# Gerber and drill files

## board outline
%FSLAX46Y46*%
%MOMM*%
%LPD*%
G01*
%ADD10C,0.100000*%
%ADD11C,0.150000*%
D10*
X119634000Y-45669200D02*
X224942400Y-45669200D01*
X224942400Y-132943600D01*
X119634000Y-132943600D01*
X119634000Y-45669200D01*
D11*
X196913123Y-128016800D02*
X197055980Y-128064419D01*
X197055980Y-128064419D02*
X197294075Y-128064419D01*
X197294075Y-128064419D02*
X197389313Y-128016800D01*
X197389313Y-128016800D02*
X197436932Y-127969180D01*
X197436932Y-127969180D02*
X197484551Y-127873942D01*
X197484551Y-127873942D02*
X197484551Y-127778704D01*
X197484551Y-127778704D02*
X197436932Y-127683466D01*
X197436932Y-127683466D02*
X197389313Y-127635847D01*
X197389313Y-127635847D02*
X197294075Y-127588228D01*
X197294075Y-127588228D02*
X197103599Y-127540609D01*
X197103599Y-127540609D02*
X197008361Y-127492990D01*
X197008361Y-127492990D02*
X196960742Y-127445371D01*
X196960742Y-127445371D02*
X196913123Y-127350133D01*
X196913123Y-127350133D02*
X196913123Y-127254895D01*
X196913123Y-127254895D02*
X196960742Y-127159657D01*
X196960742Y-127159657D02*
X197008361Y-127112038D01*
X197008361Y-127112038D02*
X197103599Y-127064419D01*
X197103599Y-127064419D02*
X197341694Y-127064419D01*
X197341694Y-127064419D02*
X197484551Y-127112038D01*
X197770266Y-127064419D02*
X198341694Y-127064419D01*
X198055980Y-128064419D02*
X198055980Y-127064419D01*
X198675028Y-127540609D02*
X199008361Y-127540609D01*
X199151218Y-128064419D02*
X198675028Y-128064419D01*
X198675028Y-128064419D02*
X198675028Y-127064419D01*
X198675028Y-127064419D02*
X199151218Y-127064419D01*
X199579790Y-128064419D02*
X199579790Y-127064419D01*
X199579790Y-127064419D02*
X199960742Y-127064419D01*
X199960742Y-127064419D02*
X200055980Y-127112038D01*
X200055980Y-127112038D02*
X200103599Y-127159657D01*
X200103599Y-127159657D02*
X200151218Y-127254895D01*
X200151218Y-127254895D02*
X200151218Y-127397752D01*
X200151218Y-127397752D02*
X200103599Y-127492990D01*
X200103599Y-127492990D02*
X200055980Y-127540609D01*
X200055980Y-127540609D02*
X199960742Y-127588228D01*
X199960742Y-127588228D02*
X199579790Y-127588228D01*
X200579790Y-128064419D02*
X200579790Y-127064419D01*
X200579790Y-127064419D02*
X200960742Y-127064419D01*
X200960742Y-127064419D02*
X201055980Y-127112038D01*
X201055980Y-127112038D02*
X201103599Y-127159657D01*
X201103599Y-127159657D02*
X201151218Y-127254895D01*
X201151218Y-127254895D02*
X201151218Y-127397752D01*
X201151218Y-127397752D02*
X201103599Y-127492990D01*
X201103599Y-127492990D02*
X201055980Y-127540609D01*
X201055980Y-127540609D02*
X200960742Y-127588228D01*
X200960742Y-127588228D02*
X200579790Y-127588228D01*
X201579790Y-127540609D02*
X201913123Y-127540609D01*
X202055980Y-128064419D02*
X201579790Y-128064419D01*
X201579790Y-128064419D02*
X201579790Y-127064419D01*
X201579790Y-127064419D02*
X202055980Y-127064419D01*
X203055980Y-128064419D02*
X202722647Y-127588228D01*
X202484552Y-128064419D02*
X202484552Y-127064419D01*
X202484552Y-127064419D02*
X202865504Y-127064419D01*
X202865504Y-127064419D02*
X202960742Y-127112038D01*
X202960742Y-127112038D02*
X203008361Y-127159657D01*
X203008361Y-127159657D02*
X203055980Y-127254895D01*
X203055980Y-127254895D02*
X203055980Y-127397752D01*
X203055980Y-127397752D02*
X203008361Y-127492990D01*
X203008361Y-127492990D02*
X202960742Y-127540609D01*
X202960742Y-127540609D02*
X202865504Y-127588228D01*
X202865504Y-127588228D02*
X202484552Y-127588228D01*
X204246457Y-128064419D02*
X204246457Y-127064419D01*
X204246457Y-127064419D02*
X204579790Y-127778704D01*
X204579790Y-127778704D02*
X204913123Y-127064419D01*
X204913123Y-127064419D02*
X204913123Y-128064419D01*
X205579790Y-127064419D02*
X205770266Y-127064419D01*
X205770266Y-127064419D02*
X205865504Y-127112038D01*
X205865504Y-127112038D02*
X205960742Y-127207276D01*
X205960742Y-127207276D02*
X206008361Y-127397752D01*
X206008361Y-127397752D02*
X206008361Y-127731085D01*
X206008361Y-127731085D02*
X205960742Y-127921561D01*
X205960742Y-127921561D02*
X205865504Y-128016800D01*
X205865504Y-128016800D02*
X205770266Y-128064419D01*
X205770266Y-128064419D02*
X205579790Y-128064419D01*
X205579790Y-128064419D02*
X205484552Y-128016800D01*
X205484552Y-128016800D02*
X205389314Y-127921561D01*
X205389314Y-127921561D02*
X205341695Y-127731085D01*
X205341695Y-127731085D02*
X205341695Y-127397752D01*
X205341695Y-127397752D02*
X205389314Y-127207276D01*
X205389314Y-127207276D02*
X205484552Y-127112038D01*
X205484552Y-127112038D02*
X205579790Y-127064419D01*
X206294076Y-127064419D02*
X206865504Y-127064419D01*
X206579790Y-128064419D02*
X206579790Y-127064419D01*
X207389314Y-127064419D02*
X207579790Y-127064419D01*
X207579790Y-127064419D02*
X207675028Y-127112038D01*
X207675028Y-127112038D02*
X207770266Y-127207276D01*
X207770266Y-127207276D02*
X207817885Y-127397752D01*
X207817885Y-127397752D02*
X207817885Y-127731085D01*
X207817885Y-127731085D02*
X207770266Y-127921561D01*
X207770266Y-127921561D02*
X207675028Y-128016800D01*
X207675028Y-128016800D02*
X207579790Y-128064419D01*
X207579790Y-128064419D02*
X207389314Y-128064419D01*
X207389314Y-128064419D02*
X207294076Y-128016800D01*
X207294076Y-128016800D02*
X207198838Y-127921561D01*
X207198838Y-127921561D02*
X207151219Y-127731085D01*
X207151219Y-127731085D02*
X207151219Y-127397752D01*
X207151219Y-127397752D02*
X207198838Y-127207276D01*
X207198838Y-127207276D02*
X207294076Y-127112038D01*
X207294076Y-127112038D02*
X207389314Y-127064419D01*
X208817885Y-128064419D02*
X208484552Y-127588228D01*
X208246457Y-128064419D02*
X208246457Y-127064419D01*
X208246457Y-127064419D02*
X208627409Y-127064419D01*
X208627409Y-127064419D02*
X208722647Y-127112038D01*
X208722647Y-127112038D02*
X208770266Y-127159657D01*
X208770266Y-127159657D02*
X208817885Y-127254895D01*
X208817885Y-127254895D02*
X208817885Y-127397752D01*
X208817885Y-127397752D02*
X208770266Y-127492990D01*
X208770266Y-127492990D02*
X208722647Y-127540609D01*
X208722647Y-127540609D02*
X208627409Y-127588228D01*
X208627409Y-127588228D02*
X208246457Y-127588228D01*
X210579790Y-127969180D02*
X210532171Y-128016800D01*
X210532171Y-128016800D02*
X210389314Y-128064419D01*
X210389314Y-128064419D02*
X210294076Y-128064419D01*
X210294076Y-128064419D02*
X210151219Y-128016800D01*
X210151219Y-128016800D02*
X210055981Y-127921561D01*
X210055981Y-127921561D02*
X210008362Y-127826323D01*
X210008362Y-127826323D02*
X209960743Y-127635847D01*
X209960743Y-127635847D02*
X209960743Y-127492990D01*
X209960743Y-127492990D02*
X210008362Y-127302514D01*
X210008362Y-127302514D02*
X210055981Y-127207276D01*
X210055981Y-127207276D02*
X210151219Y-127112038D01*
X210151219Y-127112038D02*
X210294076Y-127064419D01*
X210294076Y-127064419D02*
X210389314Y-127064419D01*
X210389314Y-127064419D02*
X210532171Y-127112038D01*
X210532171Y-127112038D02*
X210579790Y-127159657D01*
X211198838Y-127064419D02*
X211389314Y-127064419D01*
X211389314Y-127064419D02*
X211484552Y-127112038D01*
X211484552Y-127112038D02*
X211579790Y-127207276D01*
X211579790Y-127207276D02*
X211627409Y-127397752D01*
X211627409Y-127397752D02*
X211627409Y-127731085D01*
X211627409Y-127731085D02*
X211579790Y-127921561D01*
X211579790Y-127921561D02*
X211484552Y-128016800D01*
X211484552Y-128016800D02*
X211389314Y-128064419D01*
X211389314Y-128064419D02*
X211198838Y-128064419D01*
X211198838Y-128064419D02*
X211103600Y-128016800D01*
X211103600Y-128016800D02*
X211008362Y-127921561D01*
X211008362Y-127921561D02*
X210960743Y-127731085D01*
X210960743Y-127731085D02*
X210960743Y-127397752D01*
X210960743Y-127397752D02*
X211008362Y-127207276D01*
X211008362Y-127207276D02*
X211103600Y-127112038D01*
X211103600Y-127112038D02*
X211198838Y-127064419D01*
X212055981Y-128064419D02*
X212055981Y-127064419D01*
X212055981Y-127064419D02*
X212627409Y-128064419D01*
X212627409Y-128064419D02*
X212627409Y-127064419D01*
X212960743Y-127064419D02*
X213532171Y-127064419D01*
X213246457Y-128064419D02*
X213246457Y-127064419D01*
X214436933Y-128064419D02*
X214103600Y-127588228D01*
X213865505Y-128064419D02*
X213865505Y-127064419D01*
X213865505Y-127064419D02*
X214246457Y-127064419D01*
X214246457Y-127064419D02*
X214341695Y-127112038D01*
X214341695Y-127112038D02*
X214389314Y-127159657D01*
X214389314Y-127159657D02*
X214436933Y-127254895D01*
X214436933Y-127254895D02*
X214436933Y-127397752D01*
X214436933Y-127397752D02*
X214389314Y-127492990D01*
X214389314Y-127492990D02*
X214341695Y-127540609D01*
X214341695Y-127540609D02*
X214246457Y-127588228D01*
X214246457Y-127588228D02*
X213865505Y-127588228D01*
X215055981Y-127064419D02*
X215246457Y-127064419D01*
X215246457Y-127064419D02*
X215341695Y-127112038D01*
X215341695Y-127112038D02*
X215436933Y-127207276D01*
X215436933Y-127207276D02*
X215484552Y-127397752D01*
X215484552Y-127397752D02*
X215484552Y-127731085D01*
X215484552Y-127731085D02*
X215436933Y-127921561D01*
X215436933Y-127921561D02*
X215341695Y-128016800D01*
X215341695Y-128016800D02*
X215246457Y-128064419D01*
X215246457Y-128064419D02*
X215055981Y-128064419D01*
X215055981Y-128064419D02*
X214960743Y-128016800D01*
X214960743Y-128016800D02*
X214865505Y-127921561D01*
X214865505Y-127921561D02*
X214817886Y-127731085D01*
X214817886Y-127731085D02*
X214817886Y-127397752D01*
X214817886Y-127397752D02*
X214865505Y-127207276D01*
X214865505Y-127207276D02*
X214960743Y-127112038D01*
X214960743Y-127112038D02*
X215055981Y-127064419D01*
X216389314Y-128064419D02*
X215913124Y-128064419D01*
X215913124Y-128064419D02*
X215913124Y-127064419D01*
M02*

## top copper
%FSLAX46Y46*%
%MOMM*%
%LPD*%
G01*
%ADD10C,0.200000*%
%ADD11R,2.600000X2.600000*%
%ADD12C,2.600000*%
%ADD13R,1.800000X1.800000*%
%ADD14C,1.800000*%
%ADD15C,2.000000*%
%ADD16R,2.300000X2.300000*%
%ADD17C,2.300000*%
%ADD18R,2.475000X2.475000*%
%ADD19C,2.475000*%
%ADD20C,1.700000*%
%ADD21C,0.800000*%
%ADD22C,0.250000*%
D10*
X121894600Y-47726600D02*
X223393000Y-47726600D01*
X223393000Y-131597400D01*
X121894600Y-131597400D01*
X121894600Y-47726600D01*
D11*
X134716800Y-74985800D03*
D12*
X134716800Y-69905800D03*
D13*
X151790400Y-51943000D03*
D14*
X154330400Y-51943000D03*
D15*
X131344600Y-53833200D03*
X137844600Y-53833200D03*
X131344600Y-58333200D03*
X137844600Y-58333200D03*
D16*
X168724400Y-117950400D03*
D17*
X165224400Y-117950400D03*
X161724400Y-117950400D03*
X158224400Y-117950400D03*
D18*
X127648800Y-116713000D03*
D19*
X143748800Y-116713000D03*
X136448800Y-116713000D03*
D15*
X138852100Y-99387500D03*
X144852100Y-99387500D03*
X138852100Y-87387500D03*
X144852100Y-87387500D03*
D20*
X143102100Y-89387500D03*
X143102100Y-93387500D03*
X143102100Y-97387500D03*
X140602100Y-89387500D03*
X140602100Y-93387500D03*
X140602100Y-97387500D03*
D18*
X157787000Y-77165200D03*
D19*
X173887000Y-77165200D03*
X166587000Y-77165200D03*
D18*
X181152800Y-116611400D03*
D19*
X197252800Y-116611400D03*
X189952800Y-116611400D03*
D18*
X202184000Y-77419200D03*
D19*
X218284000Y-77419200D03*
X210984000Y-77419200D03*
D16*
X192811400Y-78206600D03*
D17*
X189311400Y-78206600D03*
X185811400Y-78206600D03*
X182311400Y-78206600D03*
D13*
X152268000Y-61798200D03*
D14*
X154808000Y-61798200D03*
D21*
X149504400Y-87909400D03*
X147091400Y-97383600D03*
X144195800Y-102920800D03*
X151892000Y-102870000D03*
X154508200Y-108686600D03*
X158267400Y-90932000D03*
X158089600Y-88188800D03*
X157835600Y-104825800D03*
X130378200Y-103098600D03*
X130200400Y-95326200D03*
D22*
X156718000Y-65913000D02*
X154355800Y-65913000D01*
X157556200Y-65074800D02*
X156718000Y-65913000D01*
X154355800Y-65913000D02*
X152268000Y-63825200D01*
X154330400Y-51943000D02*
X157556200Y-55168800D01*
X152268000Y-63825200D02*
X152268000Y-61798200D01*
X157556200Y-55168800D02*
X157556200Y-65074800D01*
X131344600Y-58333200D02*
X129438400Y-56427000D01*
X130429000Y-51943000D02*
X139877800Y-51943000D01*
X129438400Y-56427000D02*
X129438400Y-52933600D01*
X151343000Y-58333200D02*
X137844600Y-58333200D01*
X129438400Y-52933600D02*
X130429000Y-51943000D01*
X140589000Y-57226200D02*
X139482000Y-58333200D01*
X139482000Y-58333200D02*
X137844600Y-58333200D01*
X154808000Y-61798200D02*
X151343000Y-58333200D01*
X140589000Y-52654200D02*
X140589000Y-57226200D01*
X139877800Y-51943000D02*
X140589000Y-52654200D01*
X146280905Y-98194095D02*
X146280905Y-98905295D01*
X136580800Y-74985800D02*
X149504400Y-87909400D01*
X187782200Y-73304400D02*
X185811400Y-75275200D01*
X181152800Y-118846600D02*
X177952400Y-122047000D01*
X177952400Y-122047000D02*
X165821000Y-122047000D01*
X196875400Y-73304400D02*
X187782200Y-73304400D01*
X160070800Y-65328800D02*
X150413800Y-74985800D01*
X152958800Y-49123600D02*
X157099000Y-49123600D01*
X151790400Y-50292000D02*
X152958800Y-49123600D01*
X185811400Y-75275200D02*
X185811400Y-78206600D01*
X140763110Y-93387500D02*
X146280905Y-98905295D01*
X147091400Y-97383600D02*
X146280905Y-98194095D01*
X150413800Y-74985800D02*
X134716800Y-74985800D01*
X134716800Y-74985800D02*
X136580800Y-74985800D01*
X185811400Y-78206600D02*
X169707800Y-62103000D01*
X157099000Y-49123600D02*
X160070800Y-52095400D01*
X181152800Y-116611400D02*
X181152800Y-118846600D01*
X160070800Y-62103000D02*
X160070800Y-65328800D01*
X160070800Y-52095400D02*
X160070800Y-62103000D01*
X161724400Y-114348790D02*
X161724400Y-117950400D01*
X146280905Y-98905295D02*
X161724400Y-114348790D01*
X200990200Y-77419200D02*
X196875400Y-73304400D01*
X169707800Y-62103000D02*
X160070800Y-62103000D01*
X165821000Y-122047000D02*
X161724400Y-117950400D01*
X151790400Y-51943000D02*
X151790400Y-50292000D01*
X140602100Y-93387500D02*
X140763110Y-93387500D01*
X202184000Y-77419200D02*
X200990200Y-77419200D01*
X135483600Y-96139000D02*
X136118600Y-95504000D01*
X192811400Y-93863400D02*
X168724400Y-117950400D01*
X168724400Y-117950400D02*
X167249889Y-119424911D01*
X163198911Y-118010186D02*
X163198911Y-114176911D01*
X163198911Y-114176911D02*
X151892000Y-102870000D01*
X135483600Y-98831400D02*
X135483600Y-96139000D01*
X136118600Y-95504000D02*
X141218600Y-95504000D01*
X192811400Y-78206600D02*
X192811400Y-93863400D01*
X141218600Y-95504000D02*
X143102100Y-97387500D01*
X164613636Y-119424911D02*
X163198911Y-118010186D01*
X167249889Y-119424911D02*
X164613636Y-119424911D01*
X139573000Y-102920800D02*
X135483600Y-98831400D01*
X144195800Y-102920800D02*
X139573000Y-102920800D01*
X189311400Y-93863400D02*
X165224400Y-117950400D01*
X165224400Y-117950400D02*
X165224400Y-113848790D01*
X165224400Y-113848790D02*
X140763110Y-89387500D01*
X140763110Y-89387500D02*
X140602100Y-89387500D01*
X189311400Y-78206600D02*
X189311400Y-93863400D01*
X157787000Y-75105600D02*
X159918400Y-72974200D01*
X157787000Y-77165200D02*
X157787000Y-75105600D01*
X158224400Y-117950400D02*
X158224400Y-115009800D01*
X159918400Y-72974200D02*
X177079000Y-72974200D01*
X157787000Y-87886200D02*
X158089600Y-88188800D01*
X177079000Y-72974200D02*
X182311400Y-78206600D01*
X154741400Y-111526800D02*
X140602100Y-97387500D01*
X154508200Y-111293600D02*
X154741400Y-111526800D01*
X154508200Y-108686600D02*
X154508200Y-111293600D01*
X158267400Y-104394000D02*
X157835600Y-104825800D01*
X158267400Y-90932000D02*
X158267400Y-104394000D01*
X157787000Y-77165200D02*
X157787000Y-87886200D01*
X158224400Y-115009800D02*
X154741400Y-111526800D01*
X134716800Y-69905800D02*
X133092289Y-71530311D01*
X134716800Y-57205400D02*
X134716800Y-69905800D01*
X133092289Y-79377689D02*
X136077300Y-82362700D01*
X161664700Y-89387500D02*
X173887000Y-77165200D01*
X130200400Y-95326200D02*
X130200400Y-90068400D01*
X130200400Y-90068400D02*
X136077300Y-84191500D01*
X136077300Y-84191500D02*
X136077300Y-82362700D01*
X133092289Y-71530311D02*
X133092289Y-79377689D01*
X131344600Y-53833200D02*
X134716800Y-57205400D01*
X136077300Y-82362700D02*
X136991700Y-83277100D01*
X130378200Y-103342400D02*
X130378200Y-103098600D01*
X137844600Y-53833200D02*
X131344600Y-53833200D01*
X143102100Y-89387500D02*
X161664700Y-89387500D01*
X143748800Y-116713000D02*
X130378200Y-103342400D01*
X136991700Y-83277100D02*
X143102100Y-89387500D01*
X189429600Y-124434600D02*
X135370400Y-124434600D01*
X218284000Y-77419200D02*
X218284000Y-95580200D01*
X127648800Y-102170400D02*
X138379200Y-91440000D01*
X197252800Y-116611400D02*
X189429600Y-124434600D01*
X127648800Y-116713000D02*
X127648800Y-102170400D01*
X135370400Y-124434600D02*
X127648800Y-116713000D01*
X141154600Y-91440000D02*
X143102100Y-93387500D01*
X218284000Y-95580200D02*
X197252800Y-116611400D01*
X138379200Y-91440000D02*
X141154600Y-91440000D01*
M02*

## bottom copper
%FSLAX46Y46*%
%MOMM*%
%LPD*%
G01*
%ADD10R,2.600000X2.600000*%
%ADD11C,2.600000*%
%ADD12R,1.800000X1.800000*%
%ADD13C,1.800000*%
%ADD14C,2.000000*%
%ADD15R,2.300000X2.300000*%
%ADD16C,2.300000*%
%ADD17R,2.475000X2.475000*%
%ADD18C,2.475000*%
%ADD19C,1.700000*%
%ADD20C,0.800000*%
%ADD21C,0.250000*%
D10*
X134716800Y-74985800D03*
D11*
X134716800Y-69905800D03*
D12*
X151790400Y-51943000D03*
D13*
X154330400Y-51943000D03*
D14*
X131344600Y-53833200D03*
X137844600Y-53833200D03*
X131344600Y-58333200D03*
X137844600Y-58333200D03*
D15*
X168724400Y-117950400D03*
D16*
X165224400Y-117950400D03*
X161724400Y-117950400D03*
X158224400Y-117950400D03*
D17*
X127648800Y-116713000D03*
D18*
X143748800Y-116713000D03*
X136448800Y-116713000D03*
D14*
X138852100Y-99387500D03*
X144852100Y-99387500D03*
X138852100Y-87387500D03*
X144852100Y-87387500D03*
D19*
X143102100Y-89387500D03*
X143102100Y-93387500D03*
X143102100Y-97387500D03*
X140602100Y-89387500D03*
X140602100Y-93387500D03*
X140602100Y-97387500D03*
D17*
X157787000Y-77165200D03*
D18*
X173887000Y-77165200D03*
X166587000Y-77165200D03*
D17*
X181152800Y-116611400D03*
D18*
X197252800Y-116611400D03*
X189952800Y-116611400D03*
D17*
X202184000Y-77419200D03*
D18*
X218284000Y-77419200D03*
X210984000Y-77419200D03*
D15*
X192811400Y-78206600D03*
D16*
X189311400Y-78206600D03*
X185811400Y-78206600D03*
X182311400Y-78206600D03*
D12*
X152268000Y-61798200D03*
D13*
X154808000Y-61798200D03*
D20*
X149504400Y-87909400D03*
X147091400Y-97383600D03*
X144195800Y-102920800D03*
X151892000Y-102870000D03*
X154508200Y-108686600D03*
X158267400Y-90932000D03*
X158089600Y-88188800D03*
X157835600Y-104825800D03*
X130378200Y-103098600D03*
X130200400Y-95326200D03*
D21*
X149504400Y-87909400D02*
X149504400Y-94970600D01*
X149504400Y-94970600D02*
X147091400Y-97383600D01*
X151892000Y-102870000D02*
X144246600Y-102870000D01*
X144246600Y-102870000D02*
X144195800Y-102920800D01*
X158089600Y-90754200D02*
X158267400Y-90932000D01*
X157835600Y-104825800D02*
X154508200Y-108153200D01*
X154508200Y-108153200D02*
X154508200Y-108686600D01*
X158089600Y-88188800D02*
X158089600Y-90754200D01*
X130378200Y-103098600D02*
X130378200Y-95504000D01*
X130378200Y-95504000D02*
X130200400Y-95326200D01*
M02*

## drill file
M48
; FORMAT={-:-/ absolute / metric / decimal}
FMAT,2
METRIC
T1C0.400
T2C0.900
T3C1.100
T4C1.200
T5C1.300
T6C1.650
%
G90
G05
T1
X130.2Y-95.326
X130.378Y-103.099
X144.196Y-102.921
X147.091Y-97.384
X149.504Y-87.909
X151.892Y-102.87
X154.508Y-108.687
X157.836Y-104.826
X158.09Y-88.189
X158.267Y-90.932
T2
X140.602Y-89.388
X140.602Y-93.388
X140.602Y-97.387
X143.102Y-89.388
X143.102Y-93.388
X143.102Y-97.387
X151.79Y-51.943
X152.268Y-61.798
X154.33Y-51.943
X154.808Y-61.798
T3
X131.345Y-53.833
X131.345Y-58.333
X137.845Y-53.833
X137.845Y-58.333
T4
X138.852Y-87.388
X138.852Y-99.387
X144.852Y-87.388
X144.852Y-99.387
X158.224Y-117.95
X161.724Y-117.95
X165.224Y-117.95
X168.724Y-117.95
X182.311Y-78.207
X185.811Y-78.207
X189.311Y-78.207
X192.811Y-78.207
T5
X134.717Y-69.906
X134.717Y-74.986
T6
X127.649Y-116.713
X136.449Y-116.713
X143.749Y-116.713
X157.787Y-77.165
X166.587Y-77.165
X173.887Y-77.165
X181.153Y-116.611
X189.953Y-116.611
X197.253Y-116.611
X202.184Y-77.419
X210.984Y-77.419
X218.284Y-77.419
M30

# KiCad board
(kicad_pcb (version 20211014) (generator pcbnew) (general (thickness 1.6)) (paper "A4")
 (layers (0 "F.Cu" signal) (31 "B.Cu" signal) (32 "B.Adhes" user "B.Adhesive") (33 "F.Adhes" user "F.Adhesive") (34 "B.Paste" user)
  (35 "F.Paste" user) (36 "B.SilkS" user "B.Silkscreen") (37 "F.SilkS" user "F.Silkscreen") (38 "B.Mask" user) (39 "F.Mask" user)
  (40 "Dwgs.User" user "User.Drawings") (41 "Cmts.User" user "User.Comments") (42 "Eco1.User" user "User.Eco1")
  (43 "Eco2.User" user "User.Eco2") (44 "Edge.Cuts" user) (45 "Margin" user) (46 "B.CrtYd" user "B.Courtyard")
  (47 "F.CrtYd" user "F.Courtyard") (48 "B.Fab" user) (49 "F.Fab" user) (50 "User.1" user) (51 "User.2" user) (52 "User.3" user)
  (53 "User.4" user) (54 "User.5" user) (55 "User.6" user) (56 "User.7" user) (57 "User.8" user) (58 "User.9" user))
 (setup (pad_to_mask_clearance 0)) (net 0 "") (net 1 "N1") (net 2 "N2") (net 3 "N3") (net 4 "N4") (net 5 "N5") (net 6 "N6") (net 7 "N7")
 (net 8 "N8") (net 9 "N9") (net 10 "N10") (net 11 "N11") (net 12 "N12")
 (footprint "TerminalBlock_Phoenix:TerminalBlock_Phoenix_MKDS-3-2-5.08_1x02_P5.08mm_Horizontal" (layer "F.Cu") (at 134.7168 74.9858 90)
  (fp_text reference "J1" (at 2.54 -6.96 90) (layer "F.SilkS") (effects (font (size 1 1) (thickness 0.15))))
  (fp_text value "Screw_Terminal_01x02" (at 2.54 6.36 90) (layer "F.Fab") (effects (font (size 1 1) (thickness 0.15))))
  (pad "1" thru_hole rect (at 0 0 90) (size 2.6 2.6) (drill 1.3) (layers *.Cu *.Mask) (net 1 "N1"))
  (pad "2" thru_hole circle (at 5.08 0 90) (size 2.6 2.6) (drill 1.3) (layers *.Cu *.Mask) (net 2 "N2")))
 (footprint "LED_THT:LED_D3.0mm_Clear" (layer "F.Cu") (at 151.7904 51.943)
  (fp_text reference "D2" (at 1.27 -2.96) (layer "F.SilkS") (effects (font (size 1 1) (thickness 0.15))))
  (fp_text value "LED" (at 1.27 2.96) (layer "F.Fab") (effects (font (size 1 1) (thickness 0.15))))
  (pad "1" thru_hole rect (at 0 0) (size 1.8 1.8) (drill 0.9) (layers *.Cu *.Mask) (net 1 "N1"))
  (pad "2" thru_hole circle (at 2.54 0) (size 1.8 1.8) (drill 0.9) (layers *.Cu *.Mask) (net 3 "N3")))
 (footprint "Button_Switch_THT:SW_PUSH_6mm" (layer "F.Cu") (at 131.3446 53.8332)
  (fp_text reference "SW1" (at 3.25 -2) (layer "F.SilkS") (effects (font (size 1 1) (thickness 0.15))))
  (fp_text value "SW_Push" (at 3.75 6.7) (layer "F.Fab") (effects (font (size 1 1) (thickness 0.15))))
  (pad "1" thru_hole circle (at 0 0 90) (size 2 2) (drill 1.1) (layers *.Cu *.Mask) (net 2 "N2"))
  (pad "1" thru_hole circle (at 6.5 0 90) (size 2 2) (drill 1.1) (layers *.Cu *.Mask) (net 2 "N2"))
  (pad "2" thru_hole circle (at 0 4.5 90) (size 2 2) (drill 1.1) (layers *.Cu *.Mask) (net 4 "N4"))
  (pad "2" thru_hole circle (at 6.5 4.5 90) (size 2 2) (drill 1.1) (layers *.Cu *.Mask) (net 4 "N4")))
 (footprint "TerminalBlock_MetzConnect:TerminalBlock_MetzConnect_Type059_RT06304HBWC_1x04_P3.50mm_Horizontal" (layer "F.Cu")
  (at 168.7244 117.9504 180)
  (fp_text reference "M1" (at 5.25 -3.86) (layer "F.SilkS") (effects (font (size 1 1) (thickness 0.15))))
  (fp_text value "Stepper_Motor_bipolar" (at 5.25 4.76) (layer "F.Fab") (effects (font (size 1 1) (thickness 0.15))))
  (pad "1" thru_hole rect (at 0 0 180) (size 2.3 2.3) (drill 1.2) (layers *.Cu *.Mask) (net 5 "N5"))
  (pad "2" thru_hole circle (at 3.5 0 180) (size 2.3 2.3) (drill 1.2) (layers *.Cu *.Mask) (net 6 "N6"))
  (pad "3" thru_hole circle (at 7 0 180) (size 2.3 2.3) (drill 1.2) (layers *.Cu *.Mask) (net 1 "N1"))
  (pad "4" thru_hole circle (at 10.5 0 180) (size 2.3 2.3) (drill 1.2) (layers *.Cu *.Mask) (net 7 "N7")))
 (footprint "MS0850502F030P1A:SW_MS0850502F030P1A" (layer "F.Cu") (at 127.6488 116.713)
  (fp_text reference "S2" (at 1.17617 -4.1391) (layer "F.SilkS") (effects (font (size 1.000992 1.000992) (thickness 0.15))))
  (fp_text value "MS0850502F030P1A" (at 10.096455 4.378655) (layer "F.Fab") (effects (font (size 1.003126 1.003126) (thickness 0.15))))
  (pad "1" thru_hole rect (at 0 0) (size 2.475 2.475) (drill 1.65) (layers *.Cu *.Mask) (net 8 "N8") (solder_mask_margin 0.102))
  (pad "2" thru_hole circle (at 16.1 0) (size 2.475 2.475) (drill 1.65) (layers *.Cu *.Mask) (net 2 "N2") (solder_mask_margin 0.102))
  (pad "3" thru_hole circle (at 8.8 0) (size 2.475 2.475) (drill 1.65) (layers *.Cu *.Mask) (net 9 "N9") (solder_mask_margin 0.102)))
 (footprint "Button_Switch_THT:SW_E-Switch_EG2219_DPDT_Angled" (layer "F.Cu") (at 143.1021 89.3875 -90)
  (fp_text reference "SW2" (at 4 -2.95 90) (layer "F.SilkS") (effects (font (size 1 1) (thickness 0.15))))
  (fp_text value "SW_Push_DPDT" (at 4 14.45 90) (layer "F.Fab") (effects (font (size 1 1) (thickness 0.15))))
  (pad "" thru_hole circle (at 10 4.25 270) (size 2 2) (drill 1.2) (layers *.Cu *.Mask))
  (pad "" thru_hole circle (at 10 -1.75 270) (size 2 2) (drill 1.2) (layers *.Cu *.Mask))
  (pad "" thru_hole circle (at -2 4.25 270) (size 2 2) (drill 1.2) (layers *.Cu *.Mask))
  (pad "" thru_hole circle (at -2 -1.75 270) (size 2 2) (drill 1.2) (layers *.Cu *.Mask))
  (pad "1" thru_hole circle (at 0 0 270) (size 1.7 1.7) (drill 0.9) (layers *.Cu *.Mask) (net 2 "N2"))
  (pad "2" thru_hole circle (at 4 0 270) (size 1.7 1.7) (drill 0.9) (layers *.Cu *.Mask) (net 8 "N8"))
  (pad "3" thru_hole circle (at 8 0 270) (size 1.7 1.7) (drill 0.9) (layers *.Cu *.Mask) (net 5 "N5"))
  (pad "4" thru_hole circle (at 0 2.5 270) (size 1.7 1.7) (drill 0.9) (layers *.Cu *.Mask) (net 6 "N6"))
  (pad "5" thru_hole circle (at 4 2.5 270) (size 1.7 1.7) (drill 0.9) (layers *.Cu *.Mask) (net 1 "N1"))
  (pad "6" thru_hole circle (at 8 2.5 270) (size 1.7 1.7) (drill 0.9) (layers *.Cu *.Mask) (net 7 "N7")))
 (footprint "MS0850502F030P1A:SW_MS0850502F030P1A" (layer "F.Cu") (at 157.787 77.1652)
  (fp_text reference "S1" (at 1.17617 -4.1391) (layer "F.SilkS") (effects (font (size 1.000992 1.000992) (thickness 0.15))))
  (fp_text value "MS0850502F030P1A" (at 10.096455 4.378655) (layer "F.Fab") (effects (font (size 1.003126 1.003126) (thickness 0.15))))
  (pad "1" thru_hole rect (at 0 0) (size 2.475 2.475) (drill 1.65) (layers *.Cu *.Mask) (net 7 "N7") (solder_mask_margin 0.102))
  (pad "2" thru_hole circle (at 16.1 0) (size 2.475 2.475) (drill 1.65) (layers *.Cu *.Mask) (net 2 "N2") (solder_mask_margin 0.102))
  (pad "3" thru_hole circle (at 8.8 0) (size 2.475 2.475) (drill 1.65) (layers *.Cu *.Mask) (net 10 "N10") (solder_mask_margin 0.102)))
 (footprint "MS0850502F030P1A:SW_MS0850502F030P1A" (layer "F.Cu") (at 181.1528 116.6114)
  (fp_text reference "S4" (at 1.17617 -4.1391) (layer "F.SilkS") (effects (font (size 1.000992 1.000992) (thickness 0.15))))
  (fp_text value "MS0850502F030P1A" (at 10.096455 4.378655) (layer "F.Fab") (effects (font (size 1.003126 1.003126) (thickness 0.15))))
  (pad "1" thru_hole rect (at 0 0) (size 2.475 2.475) (drill 1.65) (layers *.Cu *.Mask) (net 1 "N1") (solder_mask_margin 0.102))
  (pad "2" thru_hole circle (at 16.1 0) (size 2.475 2.475) (drill 1.65) (layers *.Cu *.Mask) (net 8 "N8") (solder_mask_margin 0.102))
  (pad "3" thru_hole circle (at 8.8 0) (size 2.475 2.475) (drill 1.65) (layers *.Cu *.Mask) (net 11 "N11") (solder_mask_margin 0.102)))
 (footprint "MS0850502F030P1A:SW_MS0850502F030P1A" (layer "F.Cu") (at 202.184 77.4192)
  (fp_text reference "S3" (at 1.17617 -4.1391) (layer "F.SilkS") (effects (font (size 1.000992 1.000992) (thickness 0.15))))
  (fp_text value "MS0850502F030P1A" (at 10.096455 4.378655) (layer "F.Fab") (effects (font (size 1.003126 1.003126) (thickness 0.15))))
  (pad "1" thru_hole rect (at 0 0) (size 2.475 2.475) (drill 1.65) (layers *.Cu *.Mask) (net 1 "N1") (solder_mask_margin 0.102))
  (pad "2" thru_hole circle (at 16.1 0) (size 2.475 2.475) (drill 1.65) (layers *.Cu *.Mask) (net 8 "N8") (solder_mask_margin 0.102))
  (pad "3" thru_hole circle (at 8.8 0) (size 2.475 2.475) (drill 1.65) (layers *.Cu *.Mask) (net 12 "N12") (solder_mask_margin 0.102)))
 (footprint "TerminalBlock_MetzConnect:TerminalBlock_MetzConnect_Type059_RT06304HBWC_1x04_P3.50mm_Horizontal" (layer "F.Cu")
  (at 192.8114 78.2066 180)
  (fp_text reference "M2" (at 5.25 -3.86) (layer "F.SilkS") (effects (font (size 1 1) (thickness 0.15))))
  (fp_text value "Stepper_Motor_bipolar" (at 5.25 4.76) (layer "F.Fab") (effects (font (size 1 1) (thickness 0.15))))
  (pad "1" thru_hole rect (at 0 0 180) (size 2.3 2.3) (drill 1.2) (layers *.Cu *.Mask) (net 5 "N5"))
  (pad "2" thru_hole circle (at 3.5 0 180) (size 2.3 2.3) (drill 1.2) (layers *.Cu *.Mask) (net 6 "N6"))
  (pad "3" thru_hole circle (at 7 0 180) (size 2.3 2.3) (drill 1.2) (layers *.Cu *.Mask) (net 1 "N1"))
  (pad "4" thru_hole circle (at 10.5 0 180) (size 2.3 2.3) (drill 1.2) (layers *.Cu *.Mask) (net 7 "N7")))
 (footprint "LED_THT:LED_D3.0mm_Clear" (layer "F.Cu") (at 152.268 61.7982)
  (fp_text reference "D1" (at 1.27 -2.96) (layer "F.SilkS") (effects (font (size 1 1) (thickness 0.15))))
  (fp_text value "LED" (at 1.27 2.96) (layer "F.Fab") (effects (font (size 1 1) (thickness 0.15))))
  (pad "1" thru_hole rect (at 0 0) (size 1.8 1.8) (drill 0.9) (layers *.Cu *.Mask) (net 3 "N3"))
  (pad "2" thru_hole circle (at 2.54 0) (size 1.8 1.8) (drill 0.9) (layers *.Cu *.Mask) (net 4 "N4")))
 (gr_rect (start 121.8946 47.7266) (end 223.393 131.5974) (layer "F.Cu") (width 0.2) (fill none))
 (gr_rect (start 119.634 45.6692) (end 224.9424 132.9436) (layer "Edge.Cuts") (width 0.1) (fill none))
 (gr_rect (start 224.9424 132.9436) (end 224.9424 132.9436) (layer "Edge.Cuts") (width 0.1) (fill none))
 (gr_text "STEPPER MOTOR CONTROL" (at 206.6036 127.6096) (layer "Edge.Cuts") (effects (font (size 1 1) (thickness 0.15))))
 (segment (start 156.718 65.913) (end 154.3558 65.913) (width 0.25) (layer "F.Cu") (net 3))
 (segment (start 157.5562 65.0748) (end 156.718 65.913) (width 0.25) (layer "F.Cu") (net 3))
 (segment (start 154.3558 65.913) (end 152.268 63.8252) (width 0.25) (layer "F.Cu") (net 3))
 (segment (start 154.3304 51.943) (end 157.5562 55.1688) (width 0.25) (layer "F.Cu") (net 3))
 (segment (start 152.268 63.8252) (end 152.268 61.7982) (width 0.25) (layer "F.Cu") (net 3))
 (segment (start 157.5562 55.1688) (end 157.5562 65.0748) (width 0.25) (layer "F.Cu") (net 3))
 (segment (start 131.3446 58.3332) (end 129.4384 56.427) (width 0.25) (layer "F.Cu") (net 4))
 (segment (start 130.429 51.943) (end 139.8778 51.943) (width 0.25) (layer "F.Cu") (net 4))
 (segment (start 129.4384 56.427) (end 129.4384 52.9336) (width 0.25) (layer "F.Cu") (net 4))
 (segment (start 151.343 58.3332) (end 137.8446 58.3332) (width 0.25) (layer "F.Cu") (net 4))
 (segment (start 129.4384 52.9336) (end 130.429 51.943) (width 0.25) (layer "F.Cu") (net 4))
 (segment (start 140.589 57.2262) (end 139.482 58.3332) (width 0.25) (layer "F.Cu") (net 4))
 (segment (start 139.482 58.3332) (end 137.8446 58.3332) (width 0.25) (layer "F.Cu") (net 4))
 (segment (start 154.808 61.7982) (end 151.343 58.3332) (width 0.25) (layer "F.Cu") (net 4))
 (segment (start 140.589 52.6542) (end 140.589 57.2262) (width 0.25) (layer "F.Cu") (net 4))
 (segment (start 139.8778 51.943) (end 140.589 52.6542) (width 0.25) (layer "F.Cu") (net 4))
 (segment (start 146.280905 98.194095) (end 146.280905 98.905295) (width 0.25) (layer "F.Cu") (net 1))
 (segment (start 136.5808 74.9858) (end 149.5044 87.9094) (width 0.25) (layer "F.Cu") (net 1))
 (segment (start 187.7822 73.3044) (end 185.8114 75.2752) (width 0.25) (layer "F.Cu") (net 1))
 (segment (start 181.1528 118.8466) (end 177.9524 122.047) (width 0.25) (layer "F.Cu") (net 1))
 (segment (start 177.9524 122.047) (end 165.821 122.047) (width 0.25) (layer "F.Cu") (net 1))
 (segment (start 196.8754 73.3044) (end 187.7822 73.3044) (width 0.25) (layer "F.Cu") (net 1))
 (segment (start 160.0708 65.3288) (end 150.4138 74.9858) (width 0.25) (layer "F.Cu") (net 1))
 (segment (start 152.9588 49.1236) (end 157.099 49.1236) (width 0.25) (layer "F.Cu") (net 1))
 (segment (start 151.7904 50.292) (end 152.9588 49.1236) (width 0.25) (layer "F.Cu") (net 1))
 (segment (start 185.8114 75.2752) (end 185.8114 78.2066) (width 0.25) (layer "F.Cu") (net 1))
 (segment (start 140.76311 93.3875) (end 146.280905 98.905295) (width 0.25) (layer "F.Cu") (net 1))
 (segment (start 147.0914 97.3836) (end 146.280905 98.194095) (width 0.25) (layer "F.Cu") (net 1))
 (segment (start 150.4138 74.9858) (end 134.7168 74.9858) (width 0.25) (layer "F.Cu") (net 1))
 (segment (start 134.7168 74.9858) (end 136.5808 74.9858) (width 0.25) (layer "F.Cu") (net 1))
 (segment (start 185.8114 78.2066) (end 169.7078 62.103) (width 0.25) (layer "F.Cu") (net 1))
 (segment (start 157.099 49.1236) (end 160.0708 52.0954) (width 0.25) (layer "F.Cu") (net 1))
 (segment (start 181.1528 116.6114) (end 181.1528 118.8466) (width 0.25) (layer "F.Cu") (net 1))
 (segment (start 160.0708 62.103) (end 160.0708 65.3288) (width 0.25) (layer "F.Cu") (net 1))
 (segment (start 160.0708 52.0954) (end 160.0708 62.103) (width 0.25) (layer "F.Cu") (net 1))
 (segment (start 161.7244 114.34879) (end 161.7244 117.9504) (width 0.25) (layer "F.Cu") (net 1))
 (segment (start 146.280905 98.905295) (end 161.7244 114.34879) (width 0.25) (layer "F.Cu") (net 1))
 (segment (start 200.9902 77.4192) (end 196.8754 73.3044) (width 0.25) (layer "F.Cu") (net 1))
 (segment (start 169.7078 62.103) (end 160.0708 62.103) (width 0.25) (layer "F.Cu") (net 1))
 (segment (start 165.821 122.047) (end 161.7244 117.9504) (width 0.25) (layer "F.Cu") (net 1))
 (segment (start 151.7904 51.943) (end 151.7904 50.292) (width 0.25) (layer "F.Cu") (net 1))
 (segment (start 140.6021 93.3875) (end 140.76311 93.3875) (width 0.25) (layer "F.Cu") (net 1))
 (segment (start 202.184 77.4192) (end 200.9902 77.4192) (width 0.25) (layer "F.Cu") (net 1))
 (via (at 149.5044 87.9094) (size 0.8) (drill 0.4) (layers "F.Cu" "B.Cu") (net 1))
 (via (at 147.0914 97.3836) (size 0.8) (drill 0.4) (layers "F.Cu" "B.Cu") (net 1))
 (segment (start 149.5044 87.9094) (end 149.5044 94.9706) (width 0.25) (layer "B.Cu") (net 1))
 (segment (start 149.5044 94.9706) (end 147.0914 97.3836) (width 0.25) (layer "B.Cu") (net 1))
 (segment (start 135.4836 96.139) (end 136.1186 95.504) (width 0.25) (layer "F.Cu") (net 5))
 (segment (start 192.8114 93.8634) (end 168.7244 117.9504) (width 0.25) (layer "F.Cu") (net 5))
 (segment (start 168.7244 117.9504) (end 167.249889 119.424911) (width 0.25) (layer "F.Cu") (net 5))
 (segment (start 163.198911 118.010186) (end 163.198911 114.176911) (width 0.25) (layer "F.Cu") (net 5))
 (segment (start 163.198911 114.176911) (end 151.892 102.87) (width 0.25) (layer "F.Cu") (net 5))
 (segment (start 135.4836 98.8314) (end 135.4836 96.139) (width 0.25) (layer "F.Cu") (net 5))
 (segment (start 136.1186 95.504) (end 141.2186 95.504) (width 0.25) (layer "F.Cu") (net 5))
 (segment (start 192.8114 78.2066) (end 192.8114 93.8634) (width 0.25) (layer "F.Cu") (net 5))
 (segment (start 141.2186 95.504) (end 143.1021 97.3875) (width 0.25) (layer "F.Cu") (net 5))
 (segment (start 164.613636 119.424911) (end 163.198911 118.010186) (width 0.25) (layer "F.Cu") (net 5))
 (segment (start 167.249889 119.424911) (end 164.613636 119.424911) (width 0.25) (layer "F.Cu") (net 5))
 (segment (start 139.573 102.9208) (end 135.4836 98.8314) (width 0.25) (layer "F.Cu") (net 5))
 (segment (start 144.1958 102.9208) (end 139.573 102.9208) (width 0.25) (layer "F.Cu") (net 5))
 (via (at 144.1958 102.9208) (size 0.8) (drill 0.4) (layers "F.Cu" "B.Cu") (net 5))
 (via (at 151.892 102.87) (size 0.8) (drill 0.4) (layers "F.Cu" "B.Cu") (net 5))
 (segment (start 151.892 102.87) (end 144.2466 102.87) (width 0.25) (layer "B.Cu") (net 5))
 (segment (start 144.2466 102.87) (end 144.1958 102.9208) (width 0.25) (layer "B.Cu") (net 5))
 (segment (start 189.3114 93.8634) (end 165.2244 117.9504) (width 0.25) (layer "F.Cu") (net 6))
 (segment (start 165.2244 117.9504) (end 165.2244 113.84879) (width 0.25) (layer "F.Cu") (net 6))
 (segment (start 165.2244 113.84879) (end 140.76311 89.3875) (width 0.25) (layer "F.Cu") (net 6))
 (segment (start 140.76311 89.3875) (end 140.6021 89.3875) (width 0.25) (layer "F.Cu") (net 6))
 (segment (start 189.3114 78.2066) (end 189.3114 93.8634) (width 0.25) (layer "F.Cu") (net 6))
 (segment (start 157.787 75.1056) (end 159.9184 72.9742) (width 0.25) (layer "F.Cu") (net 7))
 (segment (start 157.787 77.1652) (end 157.787 75.1056) (width 0.25) (layer "F.Cu") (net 7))
 (segment (start 158.2244 117.9504) (end 158.2244 115.0098) (width 0.25) (layer "F.Cu") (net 7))
 (segment (start 159.9184 72.9742) (end 177.079 72.9742) (width 0.25) (layer "F.Cu") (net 7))
 (segment (start 157.787 87.8862) (end 158.0896 88.1888) (width 0.25) (layer "F.Cu") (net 7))
 (segment (start 177.079 72.9742) (end 182.3114 78.2066) (width 0.25) (layer "F.Cu") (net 7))
 (segment (start 154.7414 111.5268) (end 140.6021 97.3875) (width 0.25) (layer "F.Cu") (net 7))
 (segment (start 154.5082 111.2936) (end 154.7414 111.5268) (width 0.25) (layer "F.Cu") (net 7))
 (segment (start 154.5082 108.6866) (end 154.5082 111.2936) (width 0.25) (layer "F.Cu") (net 7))
 (segment (start 158.2674 104.394) (end 157.8356 104.8258) (width 0.25) (layer "F.Cu") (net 7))
 (segment (start 158.2674 90.932) (end 158.2674 104.394) (width 0.25) (layer "F.Cu") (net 7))
 (segment (start 157.787 77.1652) (end 157.787 87.8862) (width 0.25) (layer "F.Cu") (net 7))
 (segment (start 158.2244 115.0098) (end 154.7414 111.5268) (width 0.25) (layer "F.Cu") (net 7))
 (via (at 154.5082 108.6866) (size 0.8) (drill 0.4) (layers "F.Cu" "B.Cu") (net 7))
 (via (at 158.2674 90.932) (size 0.8) (drill 0.4) (layers "F.Cu" "B.Cu") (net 7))
 (via (at 158.0896 88.1888) (size 0.8) (drill 0.4) (layers "F.Cu" "B.Cu") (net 7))
 (via (at 157.8356 104.8258) (size 0.8) (drill 0.4) (layers "F.Cu" "B.Cu") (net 7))
 (segment (start 158.0896 90.7542) (end 158.2674 90.932) (width 0.25) (layer "B.Cu") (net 7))
 (segment (start 157.8356 104.8258) (end 154.5082 108.1532) (width 0.25) (layer "B.Cu") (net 7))
 (segment (start 154.5082 108.1532) (end 154.5082 108.6866) (width 0.25) (layer "B.Cu") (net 7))
 (segment (start 158.0896 88.1888) (end 158.0896 90.7542) (width 0.25) (layer "B.Cu") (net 7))
 (segment (start 134.7168 69.9058) (end 133.092289 71.530311) (width 0.25) (layer "F.Cu") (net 2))
 (segment (start 134.7168 57.2054) (end 134.7168 69.9058) (width 0.25) (layer "F.Cu") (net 2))
 (segment (start 133.092289 79.377689) (end 136.0773 82.3627) (width 0.25) (layer "F.Cu") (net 2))
 (segment (start 161.6647 89.3875) (end 173.887 77.1652) (width 0.25) (layer "F.Cu") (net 2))
 (segment (start 130.2004 95.3262) (end 130.2004 90.0684) (width 0.25) (layer "F.Cu") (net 2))
 (segment (start 130.2004 90.0684) (end 136.0773 84.1915) (width 0.25) (layer "F.Cu") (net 2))
 (segment (start 136.0773 84.1915) (end 136.0773 82.3627) (width 0.25) (layer "F.Cu") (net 2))
 (segment (start 133.092289 71.530311) (end 133.092289 79.377689) (width 0.25) (layer "F.Cu") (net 2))
 (segment (start 131.3446 53.8332) (end 134.7168 57.2054) (width 0.25) (layer "F.Cu") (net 2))
 (segment (start 136.0773 82.3627) (end 136.9917 83.2771) (width 0.25) (layer "F.Cu") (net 2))
 (segment (start 130.3782 103.3424) (end 130.3782 103.0986) (width 0.25) (layer "F.Cu") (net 2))
 (segment (start 137.8446 53.8332) (end 131.3446 53.8332) (width 0.25) (layer "F.Cu") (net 2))
 (segment (start 143.1021 89.3875) (end 161.6647 89.3875) (width 0.25) (layer "F.Cu") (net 2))
 (segment (start 143.7488 116.713) (end 130.3782 103.3424) (width 0.25) (layer "F.Cu") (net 2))
 (segment (start 136.9917 83.2771) (end 143.1021 89.3875) (width 0.25) (layer "F.Cu") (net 2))
 (via (at 130.3782 103.0986) (size 0.8) (drill 0.4) (layers "F.Cu" "B.Cu") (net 2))
 (via (at 130.2004 95.3262) (size 0.8) (drill 0.4) (layers "F.Cu" "B.Cu") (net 2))
 (segment (start 130.3782 103.0986) (end 130.3782 95.504) (width 0.25) (layer "B.Cu") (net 2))
 (segment (start 130.3782 95.504) (end 130.2004 95.3262) (width 0.25) (layer "B.Cu") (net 2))
 (segment (start 189.4296 124.4346) (end 135.3704 124.4346) (width 0.25) (layer "F.Cu") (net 8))
 (segment (start 218.284 77.4192) (end 218.284 95.5802) (width 0.25) (layer "F.Cu") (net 8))
 (segment (start 127.6488 102.1704) (end 138.3792 91.44) (width 0.25) (layer "F.Cu") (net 8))
 (segment (start 197.2528 116.6114) (end 189.4296 124.4346) (width 0.25) (layer "F.Cu") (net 8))
 (segment (start 127.6488 116.713) (end 127.6488 102.1704) (width 0.25) (layer "F.Cu") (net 8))
 (segment (start 135.3704 124.4346) (end 127.6488 116.713) (width 0.25) (layer "F.Cu") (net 8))
 (segment (start 141.1546 91.44) (end 143.1021 93.3875) (width 0.25) (layer "F.Cu") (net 8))
 (segment (start 218.284 95.5802) (end 197.2528 116.6114) (width 0.25) (layer "F.Cu") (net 8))
 (segment (start 138.3792 91.44) (end 141.1546 91.44) (width 0.25) (layer "F.Cu") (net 8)))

